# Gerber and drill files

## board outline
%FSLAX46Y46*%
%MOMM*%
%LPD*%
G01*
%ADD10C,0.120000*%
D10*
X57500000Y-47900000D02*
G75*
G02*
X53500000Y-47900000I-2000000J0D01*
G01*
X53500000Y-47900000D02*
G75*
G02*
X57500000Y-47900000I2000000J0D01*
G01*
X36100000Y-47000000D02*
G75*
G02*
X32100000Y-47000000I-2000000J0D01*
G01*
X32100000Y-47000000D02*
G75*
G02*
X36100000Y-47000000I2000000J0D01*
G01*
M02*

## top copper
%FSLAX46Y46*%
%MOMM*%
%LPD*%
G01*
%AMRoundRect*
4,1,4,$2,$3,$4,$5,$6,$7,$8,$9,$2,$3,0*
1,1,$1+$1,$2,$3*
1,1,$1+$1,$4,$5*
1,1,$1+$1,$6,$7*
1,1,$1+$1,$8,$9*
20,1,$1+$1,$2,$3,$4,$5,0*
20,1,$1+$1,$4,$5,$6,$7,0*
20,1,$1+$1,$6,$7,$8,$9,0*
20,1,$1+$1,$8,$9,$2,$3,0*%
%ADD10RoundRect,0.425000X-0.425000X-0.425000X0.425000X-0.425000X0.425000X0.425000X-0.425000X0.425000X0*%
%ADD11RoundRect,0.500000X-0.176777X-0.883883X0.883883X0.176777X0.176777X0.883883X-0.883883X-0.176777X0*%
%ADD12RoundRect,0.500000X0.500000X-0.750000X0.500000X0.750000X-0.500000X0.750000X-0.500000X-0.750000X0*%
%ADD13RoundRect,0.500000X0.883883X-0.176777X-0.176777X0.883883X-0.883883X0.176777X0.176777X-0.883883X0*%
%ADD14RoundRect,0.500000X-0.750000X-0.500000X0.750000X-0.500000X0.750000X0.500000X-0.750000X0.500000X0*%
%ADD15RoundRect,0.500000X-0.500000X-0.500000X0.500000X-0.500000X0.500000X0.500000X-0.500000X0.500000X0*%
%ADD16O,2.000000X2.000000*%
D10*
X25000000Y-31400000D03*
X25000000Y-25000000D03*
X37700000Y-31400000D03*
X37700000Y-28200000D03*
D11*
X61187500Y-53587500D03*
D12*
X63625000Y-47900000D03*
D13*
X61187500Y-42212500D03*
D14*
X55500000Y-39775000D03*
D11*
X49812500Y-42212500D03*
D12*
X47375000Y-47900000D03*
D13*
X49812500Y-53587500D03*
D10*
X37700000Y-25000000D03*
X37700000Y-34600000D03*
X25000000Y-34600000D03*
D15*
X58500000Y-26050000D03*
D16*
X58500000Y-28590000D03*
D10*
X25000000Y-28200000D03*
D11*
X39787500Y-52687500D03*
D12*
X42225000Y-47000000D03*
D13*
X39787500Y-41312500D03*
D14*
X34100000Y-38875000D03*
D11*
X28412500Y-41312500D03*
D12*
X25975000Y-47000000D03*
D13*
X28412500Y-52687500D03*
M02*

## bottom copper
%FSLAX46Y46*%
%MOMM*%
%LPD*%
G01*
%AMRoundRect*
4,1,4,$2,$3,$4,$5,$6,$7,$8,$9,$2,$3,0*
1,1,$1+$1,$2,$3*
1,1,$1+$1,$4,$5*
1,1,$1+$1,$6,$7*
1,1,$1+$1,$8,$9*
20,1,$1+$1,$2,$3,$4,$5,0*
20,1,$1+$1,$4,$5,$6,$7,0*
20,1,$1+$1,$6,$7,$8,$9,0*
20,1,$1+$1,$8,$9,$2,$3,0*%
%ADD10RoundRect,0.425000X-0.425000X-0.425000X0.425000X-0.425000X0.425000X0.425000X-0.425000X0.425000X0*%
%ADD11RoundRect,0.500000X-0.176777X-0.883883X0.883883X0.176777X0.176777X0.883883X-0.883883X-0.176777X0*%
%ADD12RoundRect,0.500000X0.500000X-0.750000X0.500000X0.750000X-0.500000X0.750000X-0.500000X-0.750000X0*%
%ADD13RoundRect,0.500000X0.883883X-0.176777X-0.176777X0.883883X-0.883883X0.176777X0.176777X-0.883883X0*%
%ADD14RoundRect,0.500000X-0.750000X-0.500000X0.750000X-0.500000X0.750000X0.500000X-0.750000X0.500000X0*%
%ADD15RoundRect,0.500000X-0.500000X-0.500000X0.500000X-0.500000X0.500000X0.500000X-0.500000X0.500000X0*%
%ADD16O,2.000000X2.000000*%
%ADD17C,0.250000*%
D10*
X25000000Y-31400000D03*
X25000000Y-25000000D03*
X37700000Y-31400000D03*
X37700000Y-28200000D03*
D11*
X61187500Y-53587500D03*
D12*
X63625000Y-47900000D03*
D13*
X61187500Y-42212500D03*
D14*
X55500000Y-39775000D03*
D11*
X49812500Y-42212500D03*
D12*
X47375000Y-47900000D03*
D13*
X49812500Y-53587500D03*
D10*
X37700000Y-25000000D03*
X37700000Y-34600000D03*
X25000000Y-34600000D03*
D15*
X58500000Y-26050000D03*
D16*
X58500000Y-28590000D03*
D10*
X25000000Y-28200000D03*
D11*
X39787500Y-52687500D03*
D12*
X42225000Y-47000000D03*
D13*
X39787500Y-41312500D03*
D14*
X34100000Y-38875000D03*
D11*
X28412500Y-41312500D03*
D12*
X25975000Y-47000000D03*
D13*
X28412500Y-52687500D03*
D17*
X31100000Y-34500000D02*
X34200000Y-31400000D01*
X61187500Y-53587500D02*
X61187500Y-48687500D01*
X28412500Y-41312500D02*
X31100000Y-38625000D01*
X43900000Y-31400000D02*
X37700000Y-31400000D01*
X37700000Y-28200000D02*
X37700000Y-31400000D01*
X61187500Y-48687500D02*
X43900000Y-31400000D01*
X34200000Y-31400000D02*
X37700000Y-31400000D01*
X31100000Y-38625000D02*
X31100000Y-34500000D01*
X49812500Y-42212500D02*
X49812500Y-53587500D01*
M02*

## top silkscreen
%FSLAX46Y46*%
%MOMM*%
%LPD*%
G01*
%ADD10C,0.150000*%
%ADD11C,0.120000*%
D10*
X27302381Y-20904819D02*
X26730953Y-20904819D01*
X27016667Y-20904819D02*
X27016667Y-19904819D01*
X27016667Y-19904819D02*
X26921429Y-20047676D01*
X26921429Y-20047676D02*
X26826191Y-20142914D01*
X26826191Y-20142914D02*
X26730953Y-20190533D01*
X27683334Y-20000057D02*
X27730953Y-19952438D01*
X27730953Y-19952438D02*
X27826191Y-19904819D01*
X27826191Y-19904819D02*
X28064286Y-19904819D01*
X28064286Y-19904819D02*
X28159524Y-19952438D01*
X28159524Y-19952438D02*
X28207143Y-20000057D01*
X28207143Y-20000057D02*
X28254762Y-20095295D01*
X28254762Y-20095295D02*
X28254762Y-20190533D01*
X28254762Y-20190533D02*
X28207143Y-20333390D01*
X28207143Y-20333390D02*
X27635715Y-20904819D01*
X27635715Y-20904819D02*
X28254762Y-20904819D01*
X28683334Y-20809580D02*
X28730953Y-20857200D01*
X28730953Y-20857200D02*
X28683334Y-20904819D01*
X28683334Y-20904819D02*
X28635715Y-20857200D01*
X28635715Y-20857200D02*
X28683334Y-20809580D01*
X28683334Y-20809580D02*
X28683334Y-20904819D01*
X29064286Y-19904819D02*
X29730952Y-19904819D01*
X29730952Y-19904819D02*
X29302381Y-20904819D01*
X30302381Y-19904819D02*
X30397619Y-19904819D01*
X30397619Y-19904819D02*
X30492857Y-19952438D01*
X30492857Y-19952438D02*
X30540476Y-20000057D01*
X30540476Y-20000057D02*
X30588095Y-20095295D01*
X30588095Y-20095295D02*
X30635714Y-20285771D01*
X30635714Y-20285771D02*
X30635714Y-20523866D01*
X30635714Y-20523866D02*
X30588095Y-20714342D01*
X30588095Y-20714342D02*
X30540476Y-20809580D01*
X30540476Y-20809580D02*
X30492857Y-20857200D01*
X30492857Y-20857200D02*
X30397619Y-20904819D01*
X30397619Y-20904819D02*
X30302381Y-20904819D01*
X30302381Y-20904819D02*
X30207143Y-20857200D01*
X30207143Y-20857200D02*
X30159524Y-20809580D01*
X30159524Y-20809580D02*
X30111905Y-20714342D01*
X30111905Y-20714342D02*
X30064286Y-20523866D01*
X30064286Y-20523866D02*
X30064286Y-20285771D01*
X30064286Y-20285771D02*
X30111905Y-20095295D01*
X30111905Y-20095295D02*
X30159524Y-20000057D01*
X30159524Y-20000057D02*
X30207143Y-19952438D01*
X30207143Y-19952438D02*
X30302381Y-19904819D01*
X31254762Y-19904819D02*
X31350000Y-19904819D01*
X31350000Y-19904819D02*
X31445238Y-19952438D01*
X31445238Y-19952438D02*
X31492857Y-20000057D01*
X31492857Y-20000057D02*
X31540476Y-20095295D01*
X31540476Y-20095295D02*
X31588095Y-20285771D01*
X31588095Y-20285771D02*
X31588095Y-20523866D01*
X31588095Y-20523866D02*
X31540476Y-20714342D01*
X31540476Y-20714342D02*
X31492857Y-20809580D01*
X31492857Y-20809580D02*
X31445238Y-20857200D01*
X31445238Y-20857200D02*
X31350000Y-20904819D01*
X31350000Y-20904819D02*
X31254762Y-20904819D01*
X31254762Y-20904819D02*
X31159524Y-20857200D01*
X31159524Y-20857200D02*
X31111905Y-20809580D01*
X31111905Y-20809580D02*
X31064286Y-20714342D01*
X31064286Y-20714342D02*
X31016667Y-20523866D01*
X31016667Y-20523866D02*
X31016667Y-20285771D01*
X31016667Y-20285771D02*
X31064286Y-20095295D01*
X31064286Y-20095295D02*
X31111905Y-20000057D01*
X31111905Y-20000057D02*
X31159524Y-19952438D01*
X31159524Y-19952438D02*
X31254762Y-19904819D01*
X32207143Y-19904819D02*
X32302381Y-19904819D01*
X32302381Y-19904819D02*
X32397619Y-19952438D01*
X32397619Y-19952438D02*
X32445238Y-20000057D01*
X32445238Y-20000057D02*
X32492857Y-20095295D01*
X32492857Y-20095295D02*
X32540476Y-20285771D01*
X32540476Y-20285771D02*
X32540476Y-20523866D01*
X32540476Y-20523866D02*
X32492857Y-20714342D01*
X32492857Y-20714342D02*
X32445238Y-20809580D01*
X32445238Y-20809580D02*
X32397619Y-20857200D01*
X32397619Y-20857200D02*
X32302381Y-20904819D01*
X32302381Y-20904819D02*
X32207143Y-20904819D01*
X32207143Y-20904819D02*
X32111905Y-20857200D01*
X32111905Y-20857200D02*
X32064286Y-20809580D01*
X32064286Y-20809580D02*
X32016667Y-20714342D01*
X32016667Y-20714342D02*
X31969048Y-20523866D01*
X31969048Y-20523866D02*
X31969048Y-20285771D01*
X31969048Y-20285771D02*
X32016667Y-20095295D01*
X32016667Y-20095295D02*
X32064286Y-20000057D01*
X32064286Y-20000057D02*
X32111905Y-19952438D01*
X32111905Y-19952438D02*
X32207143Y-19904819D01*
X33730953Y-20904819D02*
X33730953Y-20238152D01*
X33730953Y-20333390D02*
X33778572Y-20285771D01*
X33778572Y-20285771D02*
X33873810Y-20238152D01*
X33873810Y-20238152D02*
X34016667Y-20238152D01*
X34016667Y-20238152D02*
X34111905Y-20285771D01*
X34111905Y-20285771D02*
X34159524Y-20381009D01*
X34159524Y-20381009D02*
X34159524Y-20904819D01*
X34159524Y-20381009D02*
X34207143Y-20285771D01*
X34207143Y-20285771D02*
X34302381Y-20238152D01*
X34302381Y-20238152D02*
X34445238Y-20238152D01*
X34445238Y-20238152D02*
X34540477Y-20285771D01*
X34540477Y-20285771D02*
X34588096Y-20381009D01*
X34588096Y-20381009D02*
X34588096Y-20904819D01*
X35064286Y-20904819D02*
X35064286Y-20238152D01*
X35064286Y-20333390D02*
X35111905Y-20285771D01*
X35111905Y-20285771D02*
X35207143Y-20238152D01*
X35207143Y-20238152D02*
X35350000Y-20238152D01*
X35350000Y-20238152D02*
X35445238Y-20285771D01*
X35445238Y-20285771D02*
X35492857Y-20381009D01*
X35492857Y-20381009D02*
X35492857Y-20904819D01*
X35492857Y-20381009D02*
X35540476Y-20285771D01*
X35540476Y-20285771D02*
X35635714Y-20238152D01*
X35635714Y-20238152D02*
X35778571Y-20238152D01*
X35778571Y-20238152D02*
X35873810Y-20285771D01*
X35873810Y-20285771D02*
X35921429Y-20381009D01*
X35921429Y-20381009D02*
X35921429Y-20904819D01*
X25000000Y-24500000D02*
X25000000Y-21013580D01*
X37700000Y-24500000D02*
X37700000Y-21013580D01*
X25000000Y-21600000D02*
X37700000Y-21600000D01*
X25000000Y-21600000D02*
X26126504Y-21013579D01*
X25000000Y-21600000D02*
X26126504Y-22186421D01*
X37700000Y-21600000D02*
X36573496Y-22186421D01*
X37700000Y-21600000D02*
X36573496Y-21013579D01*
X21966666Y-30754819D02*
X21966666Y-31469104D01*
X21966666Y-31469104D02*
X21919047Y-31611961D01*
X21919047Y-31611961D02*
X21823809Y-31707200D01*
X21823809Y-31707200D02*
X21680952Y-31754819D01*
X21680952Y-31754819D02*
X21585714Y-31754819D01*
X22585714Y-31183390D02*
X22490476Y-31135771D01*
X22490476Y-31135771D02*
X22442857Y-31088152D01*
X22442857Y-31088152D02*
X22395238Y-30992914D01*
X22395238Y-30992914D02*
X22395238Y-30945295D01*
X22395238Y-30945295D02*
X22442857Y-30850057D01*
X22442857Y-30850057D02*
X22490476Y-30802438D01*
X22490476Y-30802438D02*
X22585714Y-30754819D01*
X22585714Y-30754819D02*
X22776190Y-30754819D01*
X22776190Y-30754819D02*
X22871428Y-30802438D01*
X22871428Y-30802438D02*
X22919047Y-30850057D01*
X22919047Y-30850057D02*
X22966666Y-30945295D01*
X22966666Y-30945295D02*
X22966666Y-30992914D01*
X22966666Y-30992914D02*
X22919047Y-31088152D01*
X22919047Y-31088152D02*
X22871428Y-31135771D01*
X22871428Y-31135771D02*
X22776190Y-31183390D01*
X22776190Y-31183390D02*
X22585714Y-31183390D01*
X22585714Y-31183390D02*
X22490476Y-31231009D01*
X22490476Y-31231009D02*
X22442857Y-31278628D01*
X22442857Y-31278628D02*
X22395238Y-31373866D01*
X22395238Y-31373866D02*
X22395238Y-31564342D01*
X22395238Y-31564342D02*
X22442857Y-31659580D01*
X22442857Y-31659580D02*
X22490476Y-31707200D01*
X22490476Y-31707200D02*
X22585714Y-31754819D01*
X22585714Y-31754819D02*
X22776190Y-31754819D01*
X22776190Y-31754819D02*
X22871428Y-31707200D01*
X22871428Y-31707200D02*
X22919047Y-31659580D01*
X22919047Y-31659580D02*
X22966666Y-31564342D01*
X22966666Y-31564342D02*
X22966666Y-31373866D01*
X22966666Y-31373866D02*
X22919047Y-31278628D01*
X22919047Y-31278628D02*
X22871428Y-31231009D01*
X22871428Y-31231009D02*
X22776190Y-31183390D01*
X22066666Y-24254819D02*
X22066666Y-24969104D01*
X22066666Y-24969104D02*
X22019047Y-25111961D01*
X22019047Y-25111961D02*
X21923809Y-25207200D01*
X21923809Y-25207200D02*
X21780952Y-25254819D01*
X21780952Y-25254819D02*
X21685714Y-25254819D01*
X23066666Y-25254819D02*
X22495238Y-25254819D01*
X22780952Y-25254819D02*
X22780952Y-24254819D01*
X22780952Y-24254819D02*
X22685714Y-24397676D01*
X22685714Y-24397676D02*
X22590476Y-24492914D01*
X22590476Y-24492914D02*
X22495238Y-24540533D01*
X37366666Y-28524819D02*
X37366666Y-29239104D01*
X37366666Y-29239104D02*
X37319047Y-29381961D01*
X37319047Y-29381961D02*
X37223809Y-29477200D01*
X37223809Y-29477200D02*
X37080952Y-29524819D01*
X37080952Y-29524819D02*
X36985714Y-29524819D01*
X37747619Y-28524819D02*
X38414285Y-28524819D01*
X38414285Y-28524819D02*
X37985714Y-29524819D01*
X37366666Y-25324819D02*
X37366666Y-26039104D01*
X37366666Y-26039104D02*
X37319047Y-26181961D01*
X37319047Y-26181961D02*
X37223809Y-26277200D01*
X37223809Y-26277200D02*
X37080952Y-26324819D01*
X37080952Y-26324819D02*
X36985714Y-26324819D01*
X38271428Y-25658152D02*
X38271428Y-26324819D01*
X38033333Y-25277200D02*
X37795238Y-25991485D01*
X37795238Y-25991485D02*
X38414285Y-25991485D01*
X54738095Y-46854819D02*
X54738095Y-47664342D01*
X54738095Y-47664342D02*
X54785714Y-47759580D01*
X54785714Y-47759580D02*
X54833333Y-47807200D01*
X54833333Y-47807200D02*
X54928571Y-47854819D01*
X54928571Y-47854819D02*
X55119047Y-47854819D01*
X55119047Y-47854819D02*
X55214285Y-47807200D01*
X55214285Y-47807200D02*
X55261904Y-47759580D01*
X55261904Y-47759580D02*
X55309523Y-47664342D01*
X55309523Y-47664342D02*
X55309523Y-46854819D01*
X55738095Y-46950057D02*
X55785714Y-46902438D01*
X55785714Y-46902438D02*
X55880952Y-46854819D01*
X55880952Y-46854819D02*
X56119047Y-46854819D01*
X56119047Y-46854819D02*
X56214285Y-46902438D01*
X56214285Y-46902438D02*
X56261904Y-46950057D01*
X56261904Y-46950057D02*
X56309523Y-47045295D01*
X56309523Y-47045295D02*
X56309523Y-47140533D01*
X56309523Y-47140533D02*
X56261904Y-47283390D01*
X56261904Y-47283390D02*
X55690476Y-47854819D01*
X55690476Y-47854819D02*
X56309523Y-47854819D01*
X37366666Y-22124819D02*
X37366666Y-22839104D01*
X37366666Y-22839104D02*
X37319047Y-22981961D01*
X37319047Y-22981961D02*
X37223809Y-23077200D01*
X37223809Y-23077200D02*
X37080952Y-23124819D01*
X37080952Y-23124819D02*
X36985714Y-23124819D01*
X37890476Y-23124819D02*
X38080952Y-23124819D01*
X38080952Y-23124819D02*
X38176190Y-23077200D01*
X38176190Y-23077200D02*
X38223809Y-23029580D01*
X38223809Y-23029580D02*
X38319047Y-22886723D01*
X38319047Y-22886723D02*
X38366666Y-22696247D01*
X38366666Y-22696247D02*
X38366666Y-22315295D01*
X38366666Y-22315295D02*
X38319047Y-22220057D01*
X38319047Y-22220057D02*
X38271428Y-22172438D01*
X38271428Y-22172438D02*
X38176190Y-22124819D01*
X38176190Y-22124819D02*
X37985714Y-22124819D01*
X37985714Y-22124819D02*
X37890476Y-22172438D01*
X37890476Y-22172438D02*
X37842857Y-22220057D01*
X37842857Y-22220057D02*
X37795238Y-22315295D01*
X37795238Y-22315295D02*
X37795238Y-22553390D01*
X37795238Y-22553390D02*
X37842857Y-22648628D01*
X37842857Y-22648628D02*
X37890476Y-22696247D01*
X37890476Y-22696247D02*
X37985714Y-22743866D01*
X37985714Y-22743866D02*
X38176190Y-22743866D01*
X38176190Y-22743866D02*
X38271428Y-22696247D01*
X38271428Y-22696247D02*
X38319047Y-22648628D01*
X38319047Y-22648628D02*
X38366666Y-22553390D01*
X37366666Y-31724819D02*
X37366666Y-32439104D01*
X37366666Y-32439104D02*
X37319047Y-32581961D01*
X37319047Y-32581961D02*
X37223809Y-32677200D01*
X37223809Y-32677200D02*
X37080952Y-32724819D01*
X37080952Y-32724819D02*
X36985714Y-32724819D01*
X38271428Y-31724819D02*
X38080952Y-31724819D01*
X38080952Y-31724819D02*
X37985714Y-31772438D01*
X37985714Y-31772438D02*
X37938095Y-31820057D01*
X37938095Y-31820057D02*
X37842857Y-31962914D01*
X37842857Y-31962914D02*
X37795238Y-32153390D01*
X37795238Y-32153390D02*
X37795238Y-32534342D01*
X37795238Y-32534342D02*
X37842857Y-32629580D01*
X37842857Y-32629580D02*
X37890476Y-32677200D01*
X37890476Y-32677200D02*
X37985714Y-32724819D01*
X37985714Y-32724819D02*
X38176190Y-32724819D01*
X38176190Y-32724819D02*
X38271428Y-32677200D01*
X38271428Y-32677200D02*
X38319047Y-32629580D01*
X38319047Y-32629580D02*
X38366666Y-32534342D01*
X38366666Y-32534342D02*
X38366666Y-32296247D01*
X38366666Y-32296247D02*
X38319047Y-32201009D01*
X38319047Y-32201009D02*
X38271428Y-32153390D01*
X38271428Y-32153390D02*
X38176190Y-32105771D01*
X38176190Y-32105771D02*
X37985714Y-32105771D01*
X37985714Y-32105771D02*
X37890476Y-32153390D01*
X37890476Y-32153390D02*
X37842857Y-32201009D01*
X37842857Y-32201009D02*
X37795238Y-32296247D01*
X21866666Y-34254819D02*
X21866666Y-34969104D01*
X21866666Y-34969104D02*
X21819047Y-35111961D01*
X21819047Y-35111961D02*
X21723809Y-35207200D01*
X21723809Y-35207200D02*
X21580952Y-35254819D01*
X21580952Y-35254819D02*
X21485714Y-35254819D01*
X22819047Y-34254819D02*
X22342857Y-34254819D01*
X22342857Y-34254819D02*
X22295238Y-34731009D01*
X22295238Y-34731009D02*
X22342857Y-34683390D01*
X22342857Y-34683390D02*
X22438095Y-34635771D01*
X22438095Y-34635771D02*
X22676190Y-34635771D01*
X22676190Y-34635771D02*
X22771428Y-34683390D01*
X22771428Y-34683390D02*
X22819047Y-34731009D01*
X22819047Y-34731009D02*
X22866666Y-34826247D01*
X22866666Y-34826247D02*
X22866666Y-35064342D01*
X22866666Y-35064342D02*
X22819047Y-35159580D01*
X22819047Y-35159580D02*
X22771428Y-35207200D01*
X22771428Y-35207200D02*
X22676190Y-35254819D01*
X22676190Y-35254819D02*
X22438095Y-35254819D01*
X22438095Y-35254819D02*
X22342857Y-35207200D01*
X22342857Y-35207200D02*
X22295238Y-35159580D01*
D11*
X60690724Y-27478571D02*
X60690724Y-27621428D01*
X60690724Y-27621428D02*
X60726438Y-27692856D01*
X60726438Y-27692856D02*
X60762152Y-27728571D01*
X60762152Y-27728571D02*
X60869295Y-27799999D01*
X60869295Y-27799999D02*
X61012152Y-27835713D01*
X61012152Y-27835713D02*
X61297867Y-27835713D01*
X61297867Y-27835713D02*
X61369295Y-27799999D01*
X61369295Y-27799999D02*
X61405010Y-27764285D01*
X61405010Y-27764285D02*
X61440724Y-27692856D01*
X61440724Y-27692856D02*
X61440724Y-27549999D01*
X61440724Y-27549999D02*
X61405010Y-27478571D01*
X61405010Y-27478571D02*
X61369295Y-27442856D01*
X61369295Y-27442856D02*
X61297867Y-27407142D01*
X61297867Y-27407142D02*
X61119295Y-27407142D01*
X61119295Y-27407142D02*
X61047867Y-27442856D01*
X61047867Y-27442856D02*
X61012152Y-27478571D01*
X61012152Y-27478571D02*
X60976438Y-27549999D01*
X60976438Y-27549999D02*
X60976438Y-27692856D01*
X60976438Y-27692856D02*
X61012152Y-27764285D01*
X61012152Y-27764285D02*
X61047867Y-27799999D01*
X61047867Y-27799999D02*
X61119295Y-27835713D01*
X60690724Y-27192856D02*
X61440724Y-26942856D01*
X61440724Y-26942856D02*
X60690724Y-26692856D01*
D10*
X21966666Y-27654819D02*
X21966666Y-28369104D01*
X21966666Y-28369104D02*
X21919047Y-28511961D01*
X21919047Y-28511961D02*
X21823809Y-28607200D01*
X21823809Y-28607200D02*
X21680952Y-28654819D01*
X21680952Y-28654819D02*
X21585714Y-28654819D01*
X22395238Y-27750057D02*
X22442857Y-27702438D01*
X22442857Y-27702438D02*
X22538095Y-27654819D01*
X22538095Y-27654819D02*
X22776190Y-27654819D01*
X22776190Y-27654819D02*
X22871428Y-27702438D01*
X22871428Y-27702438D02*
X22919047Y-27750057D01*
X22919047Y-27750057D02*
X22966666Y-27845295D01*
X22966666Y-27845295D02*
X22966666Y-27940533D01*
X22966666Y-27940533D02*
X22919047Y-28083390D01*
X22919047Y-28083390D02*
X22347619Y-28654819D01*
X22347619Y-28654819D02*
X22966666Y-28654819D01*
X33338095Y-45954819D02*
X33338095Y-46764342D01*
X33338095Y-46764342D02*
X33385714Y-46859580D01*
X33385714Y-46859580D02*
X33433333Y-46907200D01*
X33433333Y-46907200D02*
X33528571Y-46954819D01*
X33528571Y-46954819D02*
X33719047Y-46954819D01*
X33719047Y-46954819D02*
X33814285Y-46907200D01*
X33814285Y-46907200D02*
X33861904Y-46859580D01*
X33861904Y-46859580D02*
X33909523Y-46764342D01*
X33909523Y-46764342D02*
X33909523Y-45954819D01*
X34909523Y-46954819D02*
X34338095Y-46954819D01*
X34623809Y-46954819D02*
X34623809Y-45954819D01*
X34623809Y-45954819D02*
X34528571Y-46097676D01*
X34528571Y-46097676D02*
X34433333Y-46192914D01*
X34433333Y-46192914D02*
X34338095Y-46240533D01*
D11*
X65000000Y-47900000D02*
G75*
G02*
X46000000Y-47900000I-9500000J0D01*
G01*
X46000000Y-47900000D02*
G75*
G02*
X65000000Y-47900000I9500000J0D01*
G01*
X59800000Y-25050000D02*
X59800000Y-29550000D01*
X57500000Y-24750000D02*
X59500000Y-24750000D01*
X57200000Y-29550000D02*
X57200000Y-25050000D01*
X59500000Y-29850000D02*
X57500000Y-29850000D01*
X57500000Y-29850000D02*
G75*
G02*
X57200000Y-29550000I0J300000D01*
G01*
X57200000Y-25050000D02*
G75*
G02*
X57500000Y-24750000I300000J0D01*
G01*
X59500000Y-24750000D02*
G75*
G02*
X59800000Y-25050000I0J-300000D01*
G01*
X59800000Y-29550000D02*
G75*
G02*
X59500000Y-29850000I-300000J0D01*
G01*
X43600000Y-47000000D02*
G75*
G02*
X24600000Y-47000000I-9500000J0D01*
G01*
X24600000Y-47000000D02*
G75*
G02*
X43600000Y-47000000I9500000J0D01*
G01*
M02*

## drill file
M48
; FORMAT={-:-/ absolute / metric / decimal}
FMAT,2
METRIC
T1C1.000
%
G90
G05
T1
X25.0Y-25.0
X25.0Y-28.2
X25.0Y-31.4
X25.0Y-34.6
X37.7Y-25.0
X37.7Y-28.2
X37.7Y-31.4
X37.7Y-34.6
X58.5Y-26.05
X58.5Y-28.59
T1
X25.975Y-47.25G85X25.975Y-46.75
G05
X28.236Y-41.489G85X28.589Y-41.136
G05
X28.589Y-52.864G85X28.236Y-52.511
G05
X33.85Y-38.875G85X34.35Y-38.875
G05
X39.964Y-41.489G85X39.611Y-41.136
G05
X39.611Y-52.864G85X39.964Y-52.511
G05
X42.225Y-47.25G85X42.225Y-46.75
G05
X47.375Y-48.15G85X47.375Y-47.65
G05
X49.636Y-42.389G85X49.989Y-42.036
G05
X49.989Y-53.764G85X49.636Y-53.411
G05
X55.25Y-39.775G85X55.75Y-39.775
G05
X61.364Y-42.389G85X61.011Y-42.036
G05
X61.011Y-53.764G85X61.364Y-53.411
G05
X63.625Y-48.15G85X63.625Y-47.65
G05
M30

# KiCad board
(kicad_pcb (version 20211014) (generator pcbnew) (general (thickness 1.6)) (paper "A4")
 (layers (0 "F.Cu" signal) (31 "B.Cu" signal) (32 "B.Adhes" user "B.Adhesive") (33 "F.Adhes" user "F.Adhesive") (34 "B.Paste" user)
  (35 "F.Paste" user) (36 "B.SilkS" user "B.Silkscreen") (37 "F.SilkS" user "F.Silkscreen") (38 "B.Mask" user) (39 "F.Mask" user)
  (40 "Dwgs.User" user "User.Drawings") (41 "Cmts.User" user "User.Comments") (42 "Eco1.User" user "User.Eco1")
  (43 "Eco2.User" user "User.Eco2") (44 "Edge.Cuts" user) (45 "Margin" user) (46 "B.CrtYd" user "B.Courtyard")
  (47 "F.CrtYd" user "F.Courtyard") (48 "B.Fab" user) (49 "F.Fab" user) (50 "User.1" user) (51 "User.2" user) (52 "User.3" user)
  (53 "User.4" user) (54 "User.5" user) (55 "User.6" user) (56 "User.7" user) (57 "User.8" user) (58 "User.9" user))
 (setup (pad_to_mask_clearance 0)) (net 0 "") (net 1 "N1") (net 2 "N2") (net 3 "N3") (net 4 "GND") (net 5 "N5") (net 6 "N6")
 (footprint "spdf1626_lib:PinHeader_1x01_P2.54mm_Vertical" (layer "F.Cu") (at 25 31.4)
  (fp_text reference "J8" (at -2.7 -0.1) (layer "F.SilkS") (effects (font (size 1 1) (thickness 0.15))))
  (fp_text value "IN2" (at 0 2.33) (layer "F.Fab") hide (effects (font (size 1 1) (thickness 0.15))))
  (pad "1" thru_hole roundrect (at 0 0) (size 1.7 1.7) (drill 1) (layers *.Cu *.Mask) (roundrect_rratio 0.25) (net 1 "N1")))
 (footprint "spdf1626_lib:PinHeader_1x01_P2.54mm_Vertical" (layer "F.Cu") (at 25 25)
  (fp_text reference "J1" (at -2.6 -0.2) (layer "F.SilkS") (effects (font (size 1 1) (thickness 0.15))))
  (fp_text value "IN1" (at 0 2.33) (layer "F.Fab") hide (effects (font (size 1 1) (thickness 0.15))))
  (pad "1" thru_hole roundrect (at 0 0) (size 1.7 1.7) (drill 1) (layers *.Cu *.Mask) (roundrect_rratio 0.25) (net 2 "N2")))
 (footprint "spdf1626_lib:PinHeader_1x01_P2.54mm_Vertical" (layer "F.Cu") (at 37.7 31.4)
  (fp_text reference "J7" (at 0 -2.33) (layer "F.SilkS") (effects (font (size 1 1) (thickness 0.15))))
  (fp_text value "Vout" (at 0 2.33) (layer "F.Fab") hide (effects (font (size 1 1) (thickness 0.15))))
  (pad "1" thru_hole roundrect (at 0 0) (size 1.7 1.7) (drill 1) (layers *.Cu *.Mask) (roundrect_rratio 0.25) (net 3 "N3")))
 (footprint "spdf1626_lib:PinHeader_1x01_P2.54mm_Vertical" (layer "F.Cu") (at 37.7 28.2)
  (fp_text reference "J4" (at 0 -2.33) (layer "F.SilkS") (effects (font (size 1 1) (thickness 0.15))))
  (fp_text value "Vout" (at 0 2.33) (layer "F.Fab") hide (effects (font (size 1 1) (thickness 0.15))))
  (pad "1" thru_hole roundrect (at 0 0) (size 1.7 1.7) (drill 1) (layers *.Cu *.Mask) (roundrect_rratio 0.25) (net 3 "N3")))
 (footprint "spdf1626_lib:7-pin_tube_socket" (layer "F.Cu") (at 55.5 47.9)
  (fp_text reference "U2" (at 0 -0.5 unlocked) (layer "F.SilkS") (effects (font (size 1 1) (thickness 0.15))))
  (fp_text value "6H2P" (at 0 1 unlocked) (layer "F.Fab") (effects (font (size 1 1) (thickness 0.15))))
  (fp_circle (center 0 0) (end 9.5 0) (layer "F.SilkS") (width 0.12) (fill none))
  (fp_circle (center 0 0) (end 2 0) (layer "Edge.Cuts") (width 0.12) (fill none))
  (pad "1" thru_hole roundrect (at 5.6875 5.6875 45) (size 2.5 2) (drill oval 1.5 1) (layers *.Cu *.Mask) (roundrect_rratio 0.25)
   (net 3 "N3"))
  (pad "2" thru_hole roundrect (at 8.125 0 90) (size 2.5 2) (drill oval 1.5 1) (layers *.Cu *.Mask) (roundrect_rratio 0.25) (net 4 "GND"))
  (pad "3" thru_hole roundrect (at 5.6875 -5.6875 135) (size 2.5 2) (drill oval 1.5 1) (layers *.Cu *.Mask) (roundrect_rratio 0.25)
   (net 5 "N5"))
  (pad "4" thru_hole roundrect (at 0 -8.125) (size 2.5 2) (drill oval 1.5 1) (layers *.Cu *.Mask) (roundrect_rratio 0.25) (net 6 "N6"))
  (pad "5" thru_hole roundrect (at -5.6875 -5.6875 45) (size 2.5 2) (drill oval 1.5 1) (layers *.Cu *.Mask) (roundrect_rratio 0.25)
   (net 1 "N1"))
  (pad "6" thru_hole roundrect (at -8.125 0 90) (size 2.5 2) (drill oval 1.5 1) (layers *.Cu *.Mask) (roundrect_rratio 0.25) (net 4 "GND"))
  (pad "7" thru_hole roundrect (at -5.6875 5.6875 135) (size 2.5 2) (drill oval 1.5 1) (layers *.Cu *.Mask) (roundrect_rratio 0.25)
   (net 1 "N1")))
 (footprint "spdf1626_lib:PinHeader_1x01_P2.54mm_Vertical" (layer "F.Cu") (at 37.7 25)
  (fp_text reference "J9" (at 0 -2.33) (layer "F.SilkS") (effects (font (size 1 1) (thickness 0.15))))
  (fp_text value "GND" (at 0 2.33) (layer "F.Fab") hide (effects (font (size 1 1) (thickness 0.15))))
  (pad "1" thru_hole roundrect (at 0 0) (size 1.7 1.7) (drill 1) (layers *.Cu *.Mask) (roundrect_rratio 0.25) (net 4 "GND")))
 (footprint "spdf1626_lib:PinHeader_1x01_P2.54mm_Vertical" (layer "F.Cu") (at 37.7 34.6)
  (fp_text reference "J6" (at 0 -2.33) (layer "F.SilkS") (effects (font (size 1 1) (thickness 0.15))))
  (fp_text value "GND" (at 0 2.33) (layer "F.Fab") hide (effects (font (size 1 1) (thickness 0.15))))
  (pad "1" thru_hole roundrect (at 0 0) (size 1.7 1.7) (drill 1) (layers *.Cu *.Mask) (roundrect_rratio 0.25) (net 4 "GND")))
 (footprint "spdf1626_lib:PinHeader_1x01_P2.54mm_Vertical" (layer "F.Cu") (at 25 34.6)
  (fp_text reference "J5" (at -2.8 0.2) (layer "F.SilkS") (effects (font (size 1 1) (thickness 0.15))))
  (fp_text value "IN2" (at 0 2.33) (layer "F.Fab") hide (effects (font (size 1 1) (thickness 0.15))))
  (pad "1" thru_hole roundrect (at 0 0) (size 1.7 1.7) (drill 1) (layers *.Cu *.Mask) (roundrect_rratio 0.25) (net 1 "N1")))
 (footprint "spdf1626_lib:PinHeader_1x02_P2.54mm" (layer "F.Cu") (at 58.5 26.05)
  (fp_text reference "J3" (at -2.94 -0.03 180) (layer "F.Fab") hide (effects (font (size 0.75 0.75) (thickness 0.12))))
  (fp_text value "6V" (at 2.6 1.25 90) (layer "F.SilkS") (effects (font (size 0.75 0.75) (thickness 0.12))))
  (fp_line (start 1.3 -1) (end 1.3 3.5) (layer "F.SilkS") (width 0.12))
  (fp_line (start -1 -1.3) (end 1 -1.3) (layer "F.SilkS") (width 0.12))
  (fp_line (start -1.3 3.5) (end -1.3 -1) (layer "F.SilkS") (width 0.12))
  (fp_line (start 1 3.8) (end -1 3.8) (layer "F.SilkS") (width 0.12))
  (fp_arc (start -1 3.8) (mid -1.212132 3.712132) (end -1.3 3.5) (layer "F.SilkS") (width 0.12))
  (fp_arc (start -1.3 -1) (mid -1.212132 -1.212132) (end -1 -1.3) (layer "F.SilkS") (width 0.12))
  (fp_arc (start 1 -1.3) (mid 1.212132 -1.212132) (end 1.3 -1) (layer "F.SilkS") (width 0.12))
  (fp_arc (start 1.3 3.5) (mid 1.212132 3.712132) (end 1 3.8) (layer "F.SilkS") (width 0.12))
  (pad "1" thru_hole roundrect (at 0 0) (size 2 2) (drill 1) (layers *.Cu *.Mask) (roundrect_rratio 0.25) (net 6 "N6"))
  (pad "2" thru_hole oval (at 0 2.54) (size 2 2) (drill 1) (layers *.Cu *.Mask) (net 5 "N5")))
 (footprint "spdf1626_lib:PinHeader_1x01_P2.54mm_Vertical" (layer "F.Cu") (at 25 28.2)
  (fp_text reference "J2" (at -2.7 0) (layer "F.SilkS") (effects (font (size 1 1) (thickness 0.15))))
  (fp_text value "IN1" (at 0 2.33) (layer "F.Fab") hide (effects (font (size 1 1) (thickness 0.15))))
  (pad "1" thru_hole roundrect (at 0 0) (size 1.7 1.7) (drill 1) (layers *.Cu *.Mask) (roundrect_rratio 0.25) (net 2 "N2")))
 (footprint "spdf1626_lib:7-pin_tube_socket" (layer "F.Cu") (at 34.1 47)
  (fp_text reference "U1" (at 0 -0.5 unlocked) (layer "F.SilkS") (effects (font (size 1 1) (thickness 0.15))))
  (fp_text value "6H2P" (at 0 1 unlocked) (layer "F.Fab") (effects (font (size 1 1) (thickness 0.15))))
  (fp_circle (center 0 0) (end 9.5 0) (layer "F.SilkS") (width 0.12) (fill none))
  (fp_circle (center 0 0) (end 2 0) (layer "Edge.Cuts") (width 0.12) (fill none))
  (pad "1" thru_hole roundrect (at 5.6875 5.6875 45) (size 2.5 2) (drill oval 1.5 1) (layers *.Cu *.Mask) (roundrect_rratio 0.25)
   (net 2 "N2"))
  (pad "2" thru_hole roundrect (at 8.125 0 90) (size 2.5 2) (drill oval 1.5 1) (layers *.Cu *.Mask) (roundrect_rratio 0.25) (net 2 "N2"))
  (pad "3" thru_hole roundrect (at 5.6875 -5.6875 135) (size 2.5 2) (drill oval 1.5 1) (layers *.Cu *.Mask) (roundrect_rratio 0.25)
   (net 6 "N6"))
  (pad "4" thru_hole roundrect (at 0 -8.125) (size 2.5 2) (drill oval 1.5 1) (layers *.Cu *.Mask) (roundrect_rratio 0.25) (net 5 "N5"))
  (pad "5" thru_hole roundrect (at -5.6875 -5.6875 45) (size 2.5 2) (drill oval 1.5 1) (layers *.Cu *.Mask) (roundrect_rratio 0.25)
   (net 3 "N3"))
  (pad "6" thru_hole roundrect (at -8.125 0 90) (size 2.5 2) (drill oval 1.5 1) (layers *.Cu *.Mask) (roundrect_rratio 0.25) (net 4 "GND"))
  (pad "7" thru_hole roundrect (at -5.6875 5.6875 135) (size 2.5 2) (drill oval 1.5 1) (layers *.Cu *.Mask) (roundrect_rratio 0.25)
   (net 4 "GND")))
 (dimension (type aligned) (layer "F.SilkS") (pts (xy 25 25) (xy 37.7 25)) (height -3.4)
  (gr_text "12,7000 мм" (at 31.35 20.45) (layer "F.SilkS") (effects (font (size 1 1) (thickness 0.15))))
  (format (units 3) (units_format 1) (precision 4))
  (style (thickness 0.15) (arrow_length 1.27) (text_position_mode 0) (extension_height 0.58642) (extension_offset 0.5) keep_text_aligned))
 (segment (start 31.1 34.5) (end 34.2 31.4) (width 0.25) (layer "B.Cu") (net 3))
 (segment (start 61.1875 53.5875) (end 61.1875 48.6875) (width 0.25) (layer "B.Cu") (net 3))
 (segment (start 28.4125 41.3125) (end 31.1 38.625) (width 0.25) (layer "B.Cu") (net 3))
 (segment (start 43.9 31.4) (end 37.7 31.4) (width 0.25) (layer "B.Cu") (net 3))
 (segment (start 37.7 28.2) (end 37.7 31.4) (width 0.25) (layer "B.Cu") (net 3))
 (segment (start 61.1875 48.6875) (end 43.9 31.4) (width 0.25) (layer "B.Cu") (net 3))
 (segment (start 34.2 31.4) (end 37.7 31.4) (width 0.25) (layer "B.Cu") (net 3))
 (segment (start 31.1 38.625) (end 31.1 34.5) (width 0.25) (layer "B.Cu") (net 3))
 (segment (start 49.8125 42.2125) (end 49.8125 53.5875) (width 0.25) (layer "B.Cu") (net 1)))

